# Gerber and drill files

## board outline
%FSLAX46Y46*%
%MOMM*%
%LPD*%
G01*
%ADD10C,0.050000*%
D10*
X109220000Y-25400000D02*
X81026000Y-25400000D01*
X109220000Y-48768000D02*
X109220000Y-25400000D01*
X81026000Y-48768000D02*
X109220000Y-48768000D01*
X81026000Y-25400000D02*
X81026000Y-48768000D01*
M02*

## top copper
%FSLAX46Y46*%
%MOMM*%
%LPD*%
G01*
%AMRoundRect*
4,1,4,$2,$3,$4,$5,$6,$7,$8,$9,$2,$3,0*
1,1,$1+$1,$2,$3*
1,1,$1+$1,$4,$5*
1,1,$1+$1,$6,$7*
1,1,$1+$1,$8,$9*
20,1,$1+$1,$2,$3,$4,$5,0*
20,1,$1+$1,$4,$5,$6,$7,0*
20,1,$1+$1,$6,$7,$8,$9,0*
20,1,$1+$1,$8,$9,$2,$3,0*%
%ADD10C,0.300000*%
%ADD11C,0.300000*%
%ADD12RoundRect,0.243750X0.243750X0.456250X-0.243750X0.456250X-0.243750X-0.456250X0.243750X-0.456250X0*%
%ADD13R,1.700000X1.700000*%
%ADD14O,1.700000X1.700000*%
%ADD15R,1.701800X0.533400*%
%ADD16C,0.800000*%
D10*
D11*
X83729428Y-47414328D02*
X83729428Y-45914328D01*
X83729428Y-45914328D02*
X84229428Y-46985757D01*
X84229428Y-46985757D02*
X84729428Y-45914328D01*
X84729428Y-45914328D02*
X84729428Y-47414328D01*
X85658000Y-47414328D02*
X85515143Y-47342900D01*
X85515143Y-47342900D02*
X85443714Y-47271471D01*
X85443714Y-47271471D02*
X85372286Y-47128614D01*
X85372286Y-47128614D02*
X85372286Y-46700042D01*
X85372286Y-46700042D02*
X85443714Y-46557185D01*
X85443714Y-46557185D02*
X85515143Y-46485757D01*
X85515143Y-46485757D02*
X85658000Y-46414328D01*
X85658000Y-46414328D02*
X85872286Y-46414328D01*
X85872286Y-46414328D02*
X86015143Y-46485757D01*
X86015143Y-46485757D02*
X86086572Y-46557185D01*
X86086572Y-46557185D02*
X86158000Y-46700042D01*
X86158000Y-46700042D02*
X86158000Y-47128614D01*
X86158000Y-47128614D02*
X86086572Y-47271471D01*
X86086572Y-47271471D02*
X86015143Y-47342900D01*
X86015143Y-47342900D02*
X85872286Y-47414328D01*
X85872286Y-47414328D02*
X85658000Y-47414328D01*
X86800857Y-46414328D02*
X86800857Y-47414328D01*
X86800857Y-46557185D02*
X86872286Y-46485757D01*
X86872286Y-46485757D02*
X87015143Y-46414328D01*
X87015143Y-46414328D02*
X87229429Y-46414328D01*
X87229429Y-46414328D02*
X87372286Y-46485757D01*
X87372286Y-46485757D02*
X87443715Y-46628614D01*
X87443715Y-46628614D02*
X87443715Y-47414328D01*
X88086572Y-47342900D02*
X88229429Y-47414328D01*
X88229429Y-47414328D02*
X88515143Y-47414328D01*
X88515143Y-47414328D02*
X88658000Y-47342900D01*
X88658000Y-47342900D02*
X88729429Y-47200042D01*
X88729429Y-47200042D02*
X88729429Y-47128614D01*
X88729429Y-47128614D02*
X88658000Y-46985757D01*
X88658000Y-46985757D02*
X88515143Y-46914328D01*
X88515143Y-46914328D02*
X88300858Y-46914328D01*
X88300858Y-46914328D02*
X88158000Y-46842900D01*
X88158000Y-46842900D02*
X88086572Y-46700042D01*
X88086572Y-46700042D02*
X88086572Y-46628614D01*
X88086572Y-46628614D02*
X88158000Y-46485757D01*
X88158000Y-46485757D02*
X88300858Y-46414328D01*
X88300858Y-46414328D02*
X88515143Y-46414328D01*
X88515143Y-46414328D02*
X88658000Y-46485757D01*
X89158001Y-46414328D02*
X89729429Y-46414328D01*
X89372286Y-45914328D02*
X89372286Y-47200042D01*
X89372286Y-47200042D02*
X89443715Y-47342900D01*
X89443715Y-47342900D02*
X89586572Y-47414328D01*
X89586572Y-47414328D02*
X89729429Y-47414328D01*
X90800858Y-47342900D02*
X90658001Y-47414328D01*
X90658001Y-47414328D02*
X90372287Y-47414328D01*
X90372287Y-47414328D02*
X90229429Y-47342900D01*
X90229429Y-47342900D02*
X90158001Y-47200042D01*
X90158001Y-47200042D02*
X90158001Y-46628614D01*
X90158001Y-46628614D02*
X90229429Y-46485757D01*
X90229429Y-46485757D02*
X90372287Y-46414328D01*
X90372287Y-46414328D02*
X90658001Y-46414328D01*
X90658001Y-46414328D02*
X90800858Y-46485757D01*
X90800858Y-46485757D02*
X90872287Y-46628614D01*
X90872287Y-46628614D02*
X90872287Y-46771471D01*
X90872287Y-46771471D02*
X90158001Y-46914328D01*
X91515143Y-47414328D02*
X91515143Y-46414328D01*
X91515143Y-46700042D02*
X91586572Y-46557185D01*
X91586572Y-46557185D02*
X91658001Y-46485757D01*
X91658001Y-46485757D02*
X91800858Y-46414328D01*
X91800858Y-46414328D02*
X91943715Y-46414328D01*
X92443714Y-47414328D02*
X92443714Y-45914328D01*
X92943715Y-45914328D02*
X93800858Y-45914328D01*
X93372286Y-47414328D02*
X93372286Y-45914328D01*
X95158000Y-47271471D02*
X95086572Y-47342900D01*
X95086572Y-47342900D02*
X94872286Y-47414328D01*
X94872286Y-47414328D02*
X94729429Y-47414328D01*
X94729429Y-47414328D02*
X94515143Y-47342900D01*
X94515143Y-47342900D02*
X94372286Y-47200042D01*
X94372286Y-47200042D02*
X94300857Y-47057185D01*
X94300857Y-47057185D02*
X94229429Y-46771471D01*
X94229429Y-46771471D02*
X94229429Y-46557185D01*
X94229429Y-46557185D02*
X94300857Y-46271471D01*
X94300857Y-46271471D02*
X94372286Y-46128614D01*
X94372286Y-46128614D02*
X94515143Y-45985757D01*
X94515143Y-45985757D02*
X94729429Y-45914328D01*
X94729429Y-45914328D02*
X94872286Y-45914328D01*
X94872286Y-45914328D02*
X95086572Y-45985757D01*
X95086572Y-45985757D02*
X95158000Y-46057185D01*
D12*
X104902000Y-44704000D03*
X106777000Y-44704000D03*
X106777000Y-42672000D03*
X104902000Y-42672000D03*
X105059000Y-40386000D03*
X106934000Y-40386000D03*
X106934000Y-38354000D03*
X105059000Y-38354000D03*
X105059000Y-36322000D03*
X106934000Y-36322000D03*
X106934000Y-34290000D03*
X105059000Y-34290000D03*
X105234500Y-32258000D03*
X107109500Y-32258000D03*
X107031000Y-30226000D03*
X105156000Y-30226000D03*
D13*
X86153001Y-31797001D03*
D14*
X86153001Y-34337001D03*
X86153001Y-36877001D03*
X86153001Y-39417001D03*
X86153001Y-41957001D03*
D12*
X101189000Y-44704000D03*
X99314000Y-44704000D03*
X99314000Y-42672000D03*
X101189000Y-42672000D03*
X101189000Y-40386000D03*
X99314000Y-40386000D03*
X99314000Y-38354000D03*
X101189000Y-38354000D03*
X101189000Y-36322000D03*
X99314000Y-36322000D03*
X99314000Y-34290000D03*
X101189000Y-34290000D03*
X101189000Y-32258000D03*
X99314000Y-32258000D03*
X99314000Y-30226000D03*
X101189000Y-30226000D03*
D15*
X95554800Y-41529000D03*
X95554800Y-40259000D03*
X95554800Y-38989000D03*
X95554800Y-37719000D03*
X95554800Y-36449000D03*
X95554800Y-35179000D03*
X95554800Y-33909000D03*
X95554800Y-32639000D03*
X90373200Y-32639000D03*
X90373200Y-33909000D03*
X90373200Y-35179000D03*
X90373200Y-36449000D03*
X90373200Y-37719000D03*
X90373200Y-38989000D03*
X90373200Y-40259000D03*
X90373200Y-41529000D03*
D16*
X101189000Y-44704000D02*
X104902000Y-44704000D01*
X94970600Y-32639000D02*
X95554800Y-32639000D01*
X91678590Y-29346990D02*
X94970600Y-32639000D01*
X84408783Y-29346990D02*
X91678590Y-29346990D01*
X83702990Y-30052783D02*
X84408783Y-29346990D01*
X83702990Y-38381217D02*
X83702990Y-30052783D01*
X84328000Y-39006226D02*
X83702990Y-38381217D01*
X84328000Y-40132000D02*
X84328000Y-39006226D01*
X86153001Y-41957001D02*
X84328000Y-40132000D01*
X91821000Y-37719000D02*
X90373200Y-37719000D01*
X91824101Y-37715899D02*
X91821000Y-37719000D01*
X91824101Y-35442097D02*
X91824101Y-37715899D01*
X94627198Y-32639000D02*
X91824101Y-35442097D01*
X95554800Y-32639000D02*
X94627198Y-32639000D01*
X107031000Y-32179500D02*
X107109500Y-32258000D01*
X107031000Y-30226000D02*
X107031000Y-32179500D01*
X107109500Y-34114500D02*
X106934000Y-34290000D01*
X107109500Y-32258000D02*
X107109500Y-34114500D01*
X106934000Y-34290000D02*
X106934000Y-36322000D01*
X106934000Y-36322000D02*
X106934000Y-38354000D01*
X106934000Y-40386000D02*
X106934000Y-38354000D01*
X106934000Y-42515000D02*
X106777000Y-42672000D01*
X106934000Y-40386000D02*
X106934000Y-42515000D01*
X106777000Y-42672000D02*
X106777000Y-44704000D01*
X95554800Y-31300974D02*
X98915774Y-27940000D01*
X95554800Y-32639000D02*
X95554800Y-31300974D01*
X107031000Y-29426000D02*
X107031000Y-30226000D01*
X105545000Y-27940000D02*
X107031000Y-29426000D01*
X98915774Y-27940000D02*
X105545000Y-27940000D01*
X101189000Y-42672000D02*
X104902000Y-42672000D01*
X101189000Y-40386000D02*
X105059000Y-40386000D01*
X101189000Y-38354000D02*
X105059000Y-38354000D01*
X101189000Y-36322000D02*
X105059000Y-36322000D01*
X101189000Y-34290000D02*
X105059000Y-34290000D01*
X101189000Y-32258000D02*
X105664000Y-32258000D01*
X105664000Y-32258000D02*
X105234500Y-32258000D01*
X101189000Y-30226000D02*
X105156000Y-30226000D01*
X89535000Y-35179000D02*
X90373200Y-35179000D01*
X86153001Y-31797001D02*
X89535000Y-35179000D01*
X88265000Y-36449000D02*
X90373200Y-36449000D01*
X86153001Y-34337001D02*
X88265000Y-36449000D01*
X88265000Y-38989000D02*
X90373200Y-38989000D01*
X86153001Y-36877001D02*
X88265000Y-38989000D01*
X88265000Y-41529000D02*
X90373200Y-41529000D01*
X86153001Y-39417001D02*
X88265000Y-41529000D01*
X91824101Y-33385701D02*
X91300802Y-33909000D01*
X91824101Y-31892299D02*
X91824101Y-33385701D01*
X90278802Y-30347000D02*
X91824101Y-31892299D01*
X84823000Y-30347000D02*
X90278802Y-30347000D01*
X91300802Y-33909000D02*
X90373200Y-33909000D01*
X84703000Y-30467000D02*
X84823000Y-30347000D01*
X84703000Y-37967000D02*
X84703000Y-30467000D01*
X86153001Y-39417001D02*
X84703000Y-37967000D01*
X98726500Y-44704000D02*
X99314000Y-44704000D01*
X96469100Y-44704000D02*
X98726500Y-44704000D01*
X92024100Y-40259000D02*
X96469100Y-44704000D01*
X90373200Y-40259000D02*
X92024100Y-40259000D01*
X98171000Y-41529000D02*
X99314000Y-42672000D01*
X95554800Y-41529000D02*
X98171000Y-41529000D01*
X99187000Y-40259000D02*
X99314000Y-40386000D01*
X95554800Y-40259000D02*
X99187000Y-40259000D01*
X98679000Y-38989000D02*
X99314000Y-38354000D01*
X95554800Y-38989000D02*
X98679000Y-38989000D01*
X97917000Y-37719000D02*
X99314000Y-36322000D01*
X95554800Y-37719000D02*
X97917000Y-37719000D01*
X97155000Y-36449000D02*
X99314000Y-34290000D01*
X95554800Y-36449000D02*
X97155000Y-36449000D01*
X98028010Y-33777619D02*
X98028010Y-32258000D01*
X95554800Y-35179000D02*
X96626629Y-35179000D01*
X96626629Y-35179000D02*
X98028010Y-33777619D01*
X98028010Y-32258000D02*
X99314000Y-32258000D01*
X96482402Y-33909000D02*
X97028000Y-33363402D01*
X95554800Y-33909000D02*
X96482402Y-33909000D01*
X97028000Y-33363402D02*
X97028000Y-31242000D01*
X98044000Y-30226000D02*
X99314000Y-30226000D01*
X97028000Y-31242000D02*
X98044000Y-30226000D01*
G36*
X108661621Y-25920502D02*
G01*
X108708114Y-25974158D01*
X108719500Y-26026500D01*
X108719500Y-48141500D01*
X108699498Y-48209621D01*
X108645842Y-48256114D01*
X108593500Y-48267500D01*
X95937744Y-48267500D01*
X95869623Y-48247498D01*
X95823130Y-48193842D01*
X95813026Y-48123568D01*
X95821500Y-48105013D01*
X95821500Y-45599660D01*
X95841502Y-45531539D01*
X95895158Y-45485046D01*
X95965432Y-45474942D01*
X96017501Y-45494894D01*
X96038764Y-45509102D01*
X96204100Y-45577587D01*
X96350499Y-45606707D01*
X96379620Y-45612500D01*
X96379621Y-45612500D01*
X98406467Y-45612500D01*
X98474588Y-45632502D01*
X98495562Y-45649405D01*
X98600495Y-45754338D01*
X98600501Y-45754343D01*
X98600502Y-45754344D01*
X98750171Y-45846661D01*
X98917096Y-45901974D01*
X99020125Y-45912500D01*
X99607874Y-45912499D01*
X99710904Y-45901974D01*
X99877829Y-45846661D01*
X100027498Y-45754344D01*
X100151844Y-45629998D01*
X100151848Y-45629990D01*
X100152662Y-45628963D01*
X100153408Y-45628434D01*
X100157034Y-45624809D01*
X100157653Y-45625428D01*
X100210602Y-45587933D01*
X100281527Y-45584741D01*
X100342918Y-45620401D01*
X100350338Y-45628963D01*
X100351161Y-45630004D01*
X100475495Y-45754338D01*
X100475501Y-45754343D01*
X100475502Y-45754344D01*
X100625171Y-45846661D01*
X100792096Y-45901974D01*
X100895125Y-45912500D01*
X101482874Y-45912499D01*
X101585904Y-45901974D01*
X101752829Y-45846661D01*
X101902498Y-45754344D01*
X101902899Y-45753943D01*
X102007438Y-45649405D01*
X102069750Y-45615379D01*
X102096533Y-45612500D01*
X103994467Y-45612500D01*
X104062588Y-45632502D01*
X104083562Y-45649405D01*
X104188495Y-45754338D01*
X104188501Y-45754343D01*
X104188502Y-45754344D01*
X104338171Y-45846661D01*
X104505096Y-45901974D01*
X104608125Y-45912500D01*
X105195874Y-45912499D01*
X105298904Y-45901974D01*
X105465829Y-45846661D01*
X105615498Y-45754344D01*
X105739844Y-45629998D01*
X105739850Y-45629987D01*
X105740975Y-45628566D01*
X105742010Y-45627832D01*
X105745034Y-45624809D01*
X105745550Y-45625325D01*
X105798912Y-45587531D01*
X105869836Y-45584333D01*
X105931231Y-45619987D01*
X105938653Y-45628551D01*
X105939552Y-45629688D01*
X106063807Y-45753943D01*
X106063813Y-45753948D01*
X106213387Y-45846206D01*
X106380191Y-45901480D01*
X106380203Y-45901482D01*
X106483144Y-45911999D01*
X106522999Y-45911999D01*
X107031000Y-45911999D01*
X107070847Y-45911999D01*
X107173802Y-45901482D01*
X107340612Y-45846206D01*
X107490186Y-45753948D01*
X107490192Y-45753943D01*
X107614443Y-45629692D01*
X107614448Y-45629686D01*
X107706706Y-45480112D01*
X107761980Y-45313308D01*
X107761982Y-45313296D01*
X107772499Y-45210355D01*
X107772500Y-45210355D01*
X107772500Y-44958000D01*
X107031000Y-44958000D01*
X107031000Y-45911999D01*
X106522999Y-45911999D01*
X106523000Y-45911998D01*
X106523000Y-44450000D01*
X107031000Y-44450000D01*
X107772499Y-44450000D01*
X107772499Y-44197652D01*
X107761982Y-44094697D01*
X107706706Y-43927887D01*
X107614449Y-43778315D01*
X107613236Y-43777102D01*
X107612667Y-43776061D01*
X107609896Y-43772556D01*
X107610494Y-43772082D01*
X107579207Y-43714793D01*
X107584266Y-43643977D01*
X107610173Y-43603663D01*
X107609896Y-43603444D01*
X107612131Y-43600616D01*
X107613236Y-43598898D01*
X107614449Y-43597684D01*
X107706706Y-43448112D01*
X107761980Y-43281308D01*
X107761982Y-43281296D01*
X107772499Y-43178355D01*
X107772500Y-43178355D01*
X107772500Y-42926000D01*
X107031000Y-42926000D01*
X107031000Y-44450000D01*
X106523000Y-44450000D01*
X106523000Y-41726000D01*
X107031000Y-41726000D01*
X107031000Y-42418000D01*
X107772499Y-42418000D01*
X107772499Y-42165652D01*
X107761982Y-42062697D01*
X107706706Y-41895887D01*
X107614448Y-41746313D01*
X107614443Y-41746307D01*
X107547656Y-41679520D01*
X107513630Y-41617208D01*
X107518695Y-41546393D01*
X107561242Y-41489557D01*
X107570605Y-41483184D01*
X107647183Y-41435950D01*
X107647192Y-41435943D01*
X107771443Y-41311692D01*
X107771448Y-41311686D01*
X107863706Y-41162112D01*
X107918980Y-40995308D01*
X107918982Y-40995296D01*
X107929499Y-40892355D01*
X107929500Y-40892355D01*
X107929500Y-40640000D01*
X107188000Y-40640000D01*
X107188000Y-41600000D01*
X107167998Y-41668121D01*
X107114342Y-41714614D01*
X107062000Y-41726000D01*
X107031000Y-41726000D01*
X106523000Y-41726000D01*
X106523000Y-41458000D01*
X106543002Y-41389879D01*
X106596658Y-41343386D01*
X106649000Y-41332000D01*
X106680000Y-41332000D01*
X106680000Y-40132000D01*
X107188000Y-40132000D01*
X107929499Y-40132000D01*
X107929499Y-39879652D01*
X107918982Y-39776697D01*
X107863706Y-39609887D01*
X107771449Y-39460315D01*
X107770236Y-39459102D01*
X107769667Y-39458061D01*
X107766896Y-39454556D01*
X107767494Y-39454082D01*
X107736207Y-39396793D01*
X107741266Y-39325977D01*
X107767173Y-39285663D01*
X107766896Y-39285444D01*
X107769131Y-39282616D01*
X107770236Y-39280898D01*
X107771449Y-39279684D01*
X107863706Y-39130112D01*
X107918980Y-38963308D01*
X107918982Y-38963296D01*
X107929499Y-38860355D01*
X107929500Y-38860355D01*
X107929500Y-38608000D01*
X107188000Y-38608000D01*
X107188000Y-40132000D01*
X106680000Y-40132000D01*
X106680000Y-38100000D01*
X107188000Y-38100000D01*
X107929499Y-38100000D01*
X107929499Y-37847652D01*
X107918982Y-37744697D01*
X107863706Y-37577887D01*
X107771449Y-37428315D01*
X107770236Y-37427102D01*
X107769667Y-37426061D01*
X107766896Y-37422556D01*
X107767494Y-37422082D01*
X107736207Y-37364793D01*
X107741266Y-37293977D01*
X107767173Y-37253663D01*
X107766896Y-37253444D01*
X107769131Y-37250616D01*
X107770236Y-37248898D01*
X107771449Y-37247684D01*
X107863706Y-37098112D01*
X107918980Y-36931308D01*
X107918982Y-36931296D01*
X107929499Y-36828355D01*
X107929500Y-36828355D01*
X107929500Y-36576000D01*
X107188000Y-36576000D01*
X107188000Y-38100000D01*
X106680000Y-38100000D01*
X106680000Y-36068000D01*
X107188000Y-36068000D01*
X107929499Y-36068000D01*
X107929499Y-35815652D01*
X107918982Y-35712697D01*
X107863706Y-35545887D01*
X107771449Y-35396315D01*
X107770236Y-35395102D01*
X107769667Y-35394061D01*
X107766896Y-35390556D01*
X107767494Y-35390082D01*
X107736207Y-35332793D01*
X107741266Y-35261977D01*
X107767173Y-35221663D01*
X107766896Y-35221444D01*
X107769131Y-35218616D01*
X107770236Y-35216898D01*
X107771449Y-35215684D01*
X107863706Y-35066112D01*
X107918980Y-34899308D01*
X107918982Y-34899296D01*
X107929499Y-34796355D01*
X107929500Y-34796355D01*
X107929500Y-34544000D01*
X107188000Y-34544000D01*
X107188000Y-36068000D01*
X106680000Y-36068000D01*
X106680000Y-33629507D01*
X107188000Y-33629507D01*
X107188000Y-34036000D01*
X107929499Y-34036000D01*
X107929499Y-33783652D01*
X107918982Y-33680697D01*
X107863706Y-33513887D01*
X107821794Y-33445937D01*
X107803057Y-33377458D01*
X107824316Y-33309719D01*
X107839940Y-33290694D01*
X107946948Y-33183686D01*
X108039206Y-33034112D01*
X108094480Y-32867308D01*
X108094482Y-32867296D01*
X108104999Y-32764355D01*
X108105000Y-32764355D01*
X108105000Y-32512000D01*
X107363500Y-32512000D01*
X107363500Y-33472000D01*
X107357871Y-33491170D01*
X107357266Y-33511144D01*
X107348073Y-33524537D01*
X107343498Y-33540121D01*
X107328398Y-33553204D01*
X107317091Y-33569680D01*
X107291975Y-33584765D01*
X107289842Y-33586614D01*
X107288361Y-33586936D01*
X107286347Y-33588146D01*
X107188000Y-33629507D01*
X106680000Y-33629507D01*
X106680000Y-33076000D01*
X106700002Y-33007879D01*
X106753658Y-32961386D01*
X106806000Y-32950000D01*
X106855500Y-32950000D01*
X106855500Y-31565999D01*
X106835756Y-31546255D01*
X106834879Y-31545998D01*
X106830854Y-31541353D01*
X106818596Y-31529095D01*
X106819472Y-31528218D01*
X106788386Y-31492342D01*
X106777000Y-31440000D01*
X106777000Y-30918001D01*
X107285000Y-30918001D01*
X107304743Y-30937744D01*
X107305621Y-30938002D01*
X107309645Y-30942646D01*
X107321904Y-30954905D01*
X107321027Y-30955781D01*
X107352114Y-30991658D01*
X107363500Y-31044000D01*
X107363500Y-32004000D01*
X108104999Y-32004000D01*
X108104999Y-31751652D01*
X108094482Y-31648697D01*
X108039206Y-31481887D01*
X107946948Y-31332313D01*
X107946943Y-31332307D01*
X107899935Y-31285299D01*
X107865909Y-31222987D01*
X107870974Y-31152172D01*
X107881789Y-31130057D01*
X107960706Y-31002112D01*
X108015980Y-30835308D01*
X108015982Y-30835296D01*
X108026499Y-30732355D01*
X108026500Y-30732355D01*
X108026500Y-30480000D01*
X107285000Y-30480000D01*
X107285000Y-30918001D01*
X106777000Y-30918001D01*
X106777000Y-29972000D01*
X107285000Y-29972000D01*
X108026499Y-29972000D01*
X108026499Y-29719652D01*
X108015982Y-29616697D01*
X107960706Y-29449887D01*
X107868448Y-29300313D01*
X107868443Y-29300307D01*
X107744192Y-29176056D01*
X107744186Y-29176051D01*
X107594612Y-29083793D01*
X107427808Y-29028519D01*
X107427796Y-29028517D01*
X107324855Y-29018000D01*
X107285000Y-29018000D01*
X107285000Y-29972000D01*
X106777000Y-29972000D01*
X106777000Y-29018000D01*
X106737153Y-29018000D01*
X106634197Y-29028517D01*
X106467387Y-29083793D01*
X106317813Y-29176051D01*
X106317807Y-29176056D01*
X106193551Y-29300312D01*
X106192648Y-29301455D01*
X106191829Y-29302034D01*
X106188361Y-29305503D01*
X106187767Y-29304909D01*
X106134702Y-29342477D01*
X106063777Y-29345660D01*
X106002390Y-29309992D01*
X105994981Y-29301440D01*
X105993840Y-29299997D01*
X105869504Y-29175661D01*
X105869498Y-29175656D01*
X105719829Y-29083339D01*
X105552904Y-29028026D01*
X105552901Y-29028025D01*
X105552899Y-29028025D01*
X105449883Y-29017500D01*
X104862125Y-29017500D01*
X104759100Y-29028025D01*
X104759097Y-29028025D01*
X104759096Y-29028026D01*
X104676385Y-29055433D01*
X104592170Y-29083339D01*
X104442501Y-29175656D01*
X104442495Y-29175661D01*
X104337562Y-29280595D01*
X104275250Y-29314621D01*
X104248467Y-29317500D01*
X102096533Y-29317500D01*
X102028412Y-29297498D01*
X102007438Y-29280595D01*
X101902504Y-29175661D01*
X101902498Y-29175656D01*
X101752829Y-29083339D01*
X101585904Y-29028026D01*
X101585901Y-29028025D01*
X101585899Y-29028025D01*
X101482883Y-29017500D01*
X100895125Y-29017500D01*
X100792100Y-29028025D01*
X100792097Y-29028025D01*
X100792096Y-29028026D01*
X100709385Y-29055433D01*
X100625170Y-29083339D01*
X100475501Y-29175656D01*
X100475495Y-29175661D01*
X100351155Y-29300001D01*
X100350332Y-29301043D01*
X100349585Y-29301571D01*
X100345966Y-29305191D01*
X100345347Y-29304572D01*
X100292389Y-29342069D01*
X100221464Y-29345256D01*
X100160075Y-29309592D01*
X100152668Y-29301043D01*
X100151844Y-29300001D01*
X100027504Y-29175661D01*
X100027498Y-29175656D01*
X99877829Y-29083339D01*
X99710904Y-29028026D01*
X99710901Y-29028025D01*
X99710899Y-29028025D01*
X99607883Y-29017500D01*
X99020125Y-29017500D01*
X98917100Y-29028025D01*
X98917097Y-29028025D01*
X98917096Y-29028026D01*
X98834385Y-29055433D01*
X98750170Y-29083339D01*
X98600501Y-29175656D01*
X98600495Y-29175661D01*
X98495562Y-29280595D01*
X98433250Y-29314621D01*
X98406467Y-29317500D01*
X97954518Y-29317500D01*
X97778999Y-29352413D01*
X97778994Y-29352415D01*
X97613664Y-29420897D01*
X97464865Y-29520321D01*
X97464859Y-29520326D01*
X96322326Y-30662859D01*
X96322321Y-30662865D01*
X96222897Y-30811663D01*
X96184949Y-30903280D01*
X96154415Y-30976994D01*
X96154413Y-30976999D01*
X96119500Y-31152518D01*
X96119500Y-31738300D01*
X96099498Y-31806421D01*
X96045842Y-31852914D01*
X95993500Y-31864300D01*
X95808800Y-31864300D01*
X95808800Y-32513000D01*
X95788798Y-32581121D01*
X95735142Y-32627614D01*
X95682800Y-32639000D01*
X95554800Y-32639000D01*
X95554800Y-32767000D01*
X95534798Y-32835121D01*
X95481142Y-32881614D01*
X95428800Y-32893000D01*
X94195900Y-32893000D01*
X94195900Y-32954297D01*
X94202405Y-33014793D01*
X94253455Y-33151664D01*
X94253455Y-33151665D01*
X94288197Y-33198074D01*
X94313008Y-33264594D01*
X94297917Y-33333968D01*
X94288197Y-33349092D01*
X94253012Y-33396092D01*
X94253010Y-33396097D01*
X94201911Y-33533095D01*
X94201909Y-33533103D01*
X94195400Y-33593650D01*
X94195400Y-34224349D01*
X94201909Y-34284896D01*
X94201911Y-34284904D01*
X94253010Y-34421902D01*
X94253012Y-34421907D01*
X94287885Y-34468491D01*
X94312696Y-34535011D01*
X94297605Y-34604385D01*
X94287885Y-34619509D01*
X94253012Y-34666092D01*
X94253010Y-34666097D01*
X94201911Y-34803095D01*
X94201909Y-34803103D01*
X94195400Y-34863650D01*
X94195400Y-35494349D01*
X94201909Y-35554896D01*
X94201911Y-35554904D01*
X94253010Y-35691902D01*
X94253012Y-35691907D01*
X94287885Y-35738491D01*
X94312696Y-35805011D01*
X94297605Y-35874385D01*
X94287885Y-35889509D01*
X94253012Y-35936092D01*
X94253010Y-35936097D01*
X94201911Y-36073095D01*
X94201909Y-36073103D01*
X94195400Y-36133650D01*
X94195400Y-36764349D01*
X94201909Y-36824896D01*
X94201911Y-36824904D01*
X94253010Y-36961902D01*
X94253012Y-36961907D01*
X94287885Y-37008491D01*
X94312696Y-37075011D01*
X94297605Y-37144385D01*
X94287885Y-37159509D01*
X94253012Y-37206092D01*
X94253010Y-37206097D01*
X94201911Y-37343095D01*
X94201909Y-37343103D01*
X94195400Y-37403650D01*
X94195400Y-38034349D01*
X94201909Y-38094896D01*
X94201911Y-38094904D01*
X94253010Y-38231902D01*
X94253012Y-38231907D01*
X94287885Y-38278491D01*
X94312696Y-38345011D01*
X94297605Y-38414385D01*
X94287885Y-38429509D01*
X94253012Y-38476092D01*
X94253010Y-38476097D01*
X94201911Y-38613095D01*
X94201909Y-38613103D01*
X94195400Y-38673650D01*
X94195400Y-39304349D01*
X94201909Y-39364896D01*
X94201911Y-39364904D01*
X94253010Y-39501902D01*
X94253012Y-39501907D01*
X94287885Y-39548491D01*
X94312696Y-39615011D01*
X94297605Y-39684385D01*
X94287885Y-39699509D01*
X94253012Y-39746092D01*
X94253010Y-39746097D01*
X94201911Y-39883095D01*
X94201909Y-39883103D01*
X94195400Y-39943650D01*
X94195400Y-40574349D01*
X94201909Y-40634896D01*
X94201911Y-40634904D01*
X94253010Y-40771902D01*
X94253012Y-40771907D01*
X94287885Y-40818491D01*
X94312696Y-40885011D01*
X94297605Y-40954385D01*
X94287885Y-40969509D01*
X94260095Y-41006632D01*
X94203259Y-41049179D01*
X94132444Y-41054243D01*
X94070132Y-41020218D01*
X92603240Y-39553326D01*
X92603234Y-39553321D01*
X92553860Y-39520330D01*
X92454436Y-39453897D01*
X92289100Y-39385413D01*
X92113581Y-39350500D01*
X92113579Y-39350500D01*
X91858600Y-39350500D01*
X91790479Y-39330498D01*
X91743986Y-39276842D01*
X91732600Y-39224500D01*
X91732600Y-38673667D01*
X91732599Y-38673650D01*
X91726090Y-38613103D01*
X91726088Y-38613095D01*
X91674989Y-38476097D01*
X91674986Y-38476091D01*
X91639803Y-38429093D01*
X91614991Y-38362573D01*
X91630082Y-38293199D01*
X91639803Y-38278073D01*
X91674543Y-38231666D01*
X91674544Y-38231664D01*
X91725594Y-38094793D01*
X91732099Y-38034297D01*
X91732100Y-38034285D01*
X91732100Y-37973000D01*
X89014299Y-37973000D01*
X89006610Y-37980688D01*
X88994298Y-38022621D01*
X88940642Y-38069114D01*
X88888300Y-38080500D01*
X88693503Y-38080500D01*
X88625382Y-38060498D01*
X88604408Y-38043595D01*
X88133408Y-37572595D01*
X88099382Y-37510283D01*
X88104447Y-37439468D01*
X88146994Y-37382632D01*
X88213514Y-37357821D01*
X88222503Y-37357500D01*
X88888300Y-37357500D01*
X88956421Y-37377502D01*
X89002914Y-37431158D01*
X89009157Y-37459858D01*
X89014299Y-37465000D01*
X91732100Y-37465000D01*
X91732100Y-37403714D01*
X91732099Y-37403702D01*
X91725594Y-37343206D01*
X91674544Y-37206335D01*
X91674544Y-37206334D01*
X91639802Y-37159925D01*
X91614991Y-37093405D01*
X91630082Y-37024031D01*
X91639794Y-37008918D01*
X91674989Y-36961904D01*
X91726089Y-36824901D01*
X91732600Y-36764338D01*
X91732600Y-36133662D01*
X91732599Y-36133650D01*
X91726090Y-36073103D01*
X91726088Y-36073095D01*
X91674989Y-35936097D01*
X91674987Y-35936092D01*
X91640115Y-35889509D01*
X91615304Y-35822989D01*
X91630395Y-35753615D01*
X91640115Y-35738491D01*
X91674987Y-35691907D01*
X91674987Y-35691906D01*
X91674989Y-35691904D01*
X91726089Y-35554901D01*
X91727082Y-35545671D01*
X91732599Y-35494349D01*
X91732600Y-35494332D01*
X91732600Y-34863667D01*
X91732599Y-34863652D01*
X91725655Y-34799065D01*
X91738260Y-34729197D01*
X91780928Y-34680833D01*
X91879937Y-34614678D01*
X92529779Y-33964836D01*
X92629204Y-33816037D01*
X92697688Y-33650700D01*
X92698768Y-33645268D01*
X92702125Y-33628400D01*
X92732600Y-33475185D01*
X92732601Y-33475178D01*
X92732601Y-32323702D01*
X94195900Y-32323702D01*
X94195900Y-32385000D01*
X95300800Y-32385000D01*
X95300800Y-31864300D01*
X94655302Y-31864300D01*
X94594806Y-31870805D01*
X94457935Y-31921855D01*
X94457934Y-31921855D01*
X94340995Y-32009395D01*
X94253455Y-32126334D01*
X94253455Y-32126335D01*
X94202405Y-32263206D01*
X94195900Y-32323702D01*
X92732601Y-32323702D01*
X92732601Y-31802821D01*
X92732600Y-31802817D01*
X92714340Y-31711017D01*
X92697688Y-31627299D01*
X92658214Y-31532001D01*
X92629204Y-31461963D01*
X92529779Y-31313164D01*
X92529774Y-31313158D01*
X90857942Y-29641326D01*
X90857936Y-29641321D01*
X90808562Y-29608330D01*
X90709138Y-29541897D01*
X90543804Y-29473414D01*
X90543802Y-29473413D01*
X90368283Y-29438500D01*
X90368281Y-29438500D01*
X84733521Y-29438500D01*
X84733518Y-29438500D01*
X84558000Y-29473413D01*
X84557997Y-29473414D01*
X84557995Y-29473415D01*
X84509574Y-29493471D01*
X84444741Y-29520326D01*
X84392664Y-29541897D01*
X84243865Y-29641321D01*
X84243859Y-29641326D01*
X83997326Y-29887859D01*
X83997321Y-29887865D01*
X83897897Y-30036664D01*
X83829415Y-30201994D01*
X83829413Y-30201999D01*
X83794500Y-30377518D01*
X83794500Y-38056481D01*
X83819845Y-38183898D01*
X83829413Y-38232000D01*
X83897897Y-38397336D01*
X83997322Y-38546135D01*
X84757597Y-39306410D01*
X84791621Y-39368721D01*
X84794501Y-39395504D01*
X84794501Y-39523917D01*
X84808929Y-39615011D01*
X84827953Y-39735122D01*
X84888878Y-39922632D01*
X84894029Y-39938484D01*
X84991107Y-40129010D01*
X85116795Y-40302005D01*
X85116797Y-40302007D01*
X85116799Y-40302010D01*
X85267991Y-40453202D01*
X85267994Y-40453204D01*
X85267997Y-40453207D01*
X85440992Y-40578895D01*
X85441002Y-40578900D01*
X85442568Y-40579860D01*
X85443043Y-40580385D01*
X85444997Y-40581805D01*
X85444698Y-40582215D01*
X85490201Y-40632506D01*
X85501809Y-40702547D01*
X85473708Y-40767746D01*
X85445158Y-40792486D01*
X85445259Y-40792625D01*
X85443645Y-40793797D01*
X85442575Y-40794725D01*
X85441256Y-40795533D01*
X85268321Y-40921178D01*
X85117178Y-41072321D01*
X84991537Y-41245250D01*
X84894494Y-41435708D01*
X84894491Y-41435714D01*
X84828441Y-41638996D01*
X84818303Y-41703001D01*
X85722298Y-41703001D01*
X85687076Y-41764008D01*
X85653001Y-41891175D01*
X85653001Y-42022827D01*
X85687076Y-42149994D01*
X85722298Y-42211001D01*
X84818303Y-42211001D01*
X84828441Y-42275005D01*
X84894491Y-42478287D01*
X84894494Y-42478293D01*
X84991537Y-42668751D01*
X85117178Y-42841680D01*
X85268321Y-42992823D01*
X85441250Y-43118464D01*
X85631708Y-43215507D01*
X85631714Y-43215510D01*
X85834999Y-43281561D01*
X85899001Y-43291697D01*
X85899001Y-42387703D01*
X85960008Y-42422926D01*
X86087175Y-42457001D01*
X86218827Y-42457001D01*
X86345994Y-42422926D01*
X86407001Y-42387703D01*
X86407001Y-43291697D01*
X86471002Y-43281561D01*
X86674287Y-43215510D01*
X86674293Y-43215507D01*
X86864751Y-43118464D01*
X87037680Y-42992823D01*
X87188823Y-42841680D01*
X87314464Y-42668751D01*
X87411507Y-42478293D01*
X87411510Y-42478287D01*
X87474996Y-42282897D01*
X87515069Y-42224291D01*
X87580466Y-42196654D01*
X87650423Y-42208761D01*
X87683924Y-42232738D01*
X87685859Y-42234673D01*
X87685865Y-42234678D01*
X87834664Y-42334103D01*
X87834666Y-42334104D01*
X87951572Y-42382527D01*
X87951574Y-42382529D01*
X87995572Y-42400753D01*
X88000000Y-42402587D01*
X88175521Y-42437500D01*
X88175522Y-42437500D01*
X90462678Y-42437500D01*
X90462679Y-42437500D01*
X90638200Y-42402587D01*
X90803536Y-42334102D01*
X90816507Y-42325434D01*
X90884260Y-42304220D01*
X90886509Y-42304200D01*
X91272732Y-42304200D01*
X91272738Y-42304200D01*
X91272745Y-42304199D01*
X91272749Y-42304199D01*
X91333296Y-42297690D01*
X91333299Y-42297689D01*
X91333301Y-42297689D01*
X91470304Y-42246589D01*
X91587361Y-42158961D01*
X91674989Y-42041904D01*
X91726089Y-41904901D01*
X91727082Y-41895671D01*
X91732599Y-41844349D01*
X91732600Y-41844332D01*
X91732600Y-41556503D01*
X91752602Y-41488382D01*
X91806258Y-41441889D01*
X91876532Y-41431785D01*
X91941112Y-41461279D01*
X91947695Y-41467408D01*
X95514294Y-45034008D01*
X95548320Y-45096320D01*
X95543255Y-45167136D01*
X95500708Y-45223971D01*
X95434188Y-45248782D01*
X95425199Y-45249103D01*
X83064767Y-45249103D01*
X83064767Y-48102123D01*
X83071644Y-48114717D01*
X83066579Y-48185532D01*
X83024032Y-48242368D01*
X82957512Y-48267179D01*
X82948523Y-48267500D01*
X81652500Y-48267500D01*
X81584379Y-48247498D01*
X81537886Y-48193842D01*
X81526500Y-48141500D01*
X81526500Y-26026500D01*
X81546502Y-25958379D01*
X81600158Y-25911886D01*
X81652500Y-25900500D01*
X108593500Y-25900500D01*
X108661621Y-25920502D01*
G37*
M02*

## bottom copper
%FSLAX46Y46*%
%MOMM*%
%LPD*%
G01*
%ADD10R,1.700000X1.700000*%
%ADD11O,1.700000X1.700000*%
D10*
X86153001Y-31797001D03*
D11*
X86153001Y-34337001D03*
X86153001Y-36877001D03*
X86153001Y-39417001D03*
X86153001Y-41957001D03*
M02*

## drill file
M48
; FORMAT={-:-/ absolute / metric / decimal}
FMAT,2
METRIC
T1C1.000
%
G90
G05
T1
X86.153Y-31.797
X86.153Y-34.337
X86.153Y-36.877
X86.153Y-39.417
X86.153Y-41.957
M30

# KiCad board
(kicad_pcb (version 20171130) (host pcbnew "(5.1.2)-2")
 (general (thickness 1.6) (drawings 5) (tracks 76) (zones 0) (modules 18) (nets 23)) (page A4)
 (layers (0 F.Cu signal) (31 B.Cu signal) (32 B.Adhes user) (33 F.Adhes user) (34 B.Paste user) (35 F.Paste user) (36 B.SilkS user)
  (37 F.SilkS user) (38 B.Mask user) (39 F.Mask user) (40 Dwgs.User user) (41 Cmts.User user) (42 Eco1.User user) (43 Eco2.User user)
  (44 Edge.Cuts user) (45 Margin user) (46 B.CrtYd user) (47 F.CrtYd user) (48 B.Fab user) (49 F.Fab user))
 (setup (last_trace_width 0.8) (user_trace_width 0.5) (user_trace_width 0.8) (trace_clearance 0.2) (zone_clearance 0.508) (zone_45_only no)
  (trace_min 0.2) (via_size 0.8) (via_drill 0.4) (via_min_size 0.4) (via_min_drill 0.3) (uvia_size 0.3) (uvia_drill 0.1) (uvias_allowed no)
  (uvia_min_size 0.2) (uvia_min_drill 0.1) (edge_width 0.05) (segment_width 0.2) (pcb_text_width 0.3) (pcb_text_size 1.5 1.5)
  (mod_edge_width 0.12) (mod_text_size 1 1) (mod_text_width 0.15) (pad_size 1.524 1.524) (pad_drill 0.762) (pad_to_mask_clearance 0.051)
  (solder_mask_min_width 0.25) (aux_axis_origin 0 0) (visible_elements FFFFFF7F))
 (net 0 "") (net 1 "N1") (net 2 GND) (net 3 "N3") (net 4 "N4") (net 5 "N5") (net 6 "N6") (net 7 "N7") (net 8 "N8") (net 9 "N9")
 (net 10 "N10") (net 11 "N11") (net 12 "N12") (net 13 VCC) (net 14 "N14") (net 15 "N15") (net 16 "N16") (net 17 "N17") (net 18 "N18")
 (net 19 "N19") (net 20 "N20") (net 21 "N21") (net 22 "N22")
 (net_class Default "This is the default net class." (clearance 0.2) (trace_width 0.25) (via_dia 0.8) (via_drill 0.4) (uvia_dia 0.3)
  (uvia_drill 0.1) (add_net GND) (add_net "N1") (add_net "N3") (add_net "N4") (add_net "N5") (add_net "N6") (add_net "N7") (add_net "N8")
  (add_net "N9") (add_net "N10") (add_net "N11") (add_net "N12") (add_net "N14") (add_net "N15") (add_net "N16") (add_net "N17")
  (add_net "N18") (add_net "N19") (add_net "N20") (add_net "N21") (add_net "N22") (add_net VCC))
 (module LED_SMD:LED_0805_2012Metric (layer F.Cu) (at 105.8395 44.704 180)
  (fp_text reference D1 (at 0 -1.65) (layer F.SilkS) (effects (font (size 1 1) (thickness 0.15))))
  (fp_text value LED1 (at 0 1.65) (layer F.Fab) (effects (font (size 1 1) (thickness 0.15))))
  (pad 2 smd roundrect (at 0.9375 0 180) (size 0.975 1.4) (layers F.Cu F.Paste F.Mask) (roundrect_rratio 0.25) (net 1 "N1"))
  (pad 1 smd roundrect (at -0.9375 0 180) (size 0.975 1.4) (layers F.Cu F.Paste F.Mask) (roundrect_rratio 0.25) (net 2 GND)))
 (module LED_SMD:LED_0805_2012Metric (layer F.Cu) (at 105.8395 42.672 180)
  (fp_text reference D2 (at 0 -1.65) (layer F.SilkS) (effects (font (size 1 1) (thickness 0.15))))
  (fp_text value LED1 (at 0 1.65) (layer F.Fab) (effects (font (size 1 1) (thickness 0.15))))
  (pad 1 smd roundrect (at -0.9375 0 180) (size 0.975 1.4) (layers F.Cu F.Paste F.Mask) (roundrect_rratio 0.25) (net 2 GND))
  (pad 2 smd roundrect (at 0.9375 0 180) (size 0.975 1.4) (layers F.Cu F.Paste F.Mask) (roundrect_rratio 0.25) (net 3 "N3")))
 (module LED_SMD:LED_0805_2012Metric (layer F.Cu) (at 105.9965 40.386 180)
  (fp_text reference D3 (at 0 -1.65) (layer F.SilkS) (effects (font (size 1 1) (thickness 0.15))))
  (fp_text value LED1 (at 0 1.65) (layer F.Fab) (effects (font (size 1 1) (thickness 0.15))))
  (pad 2 smd roundrect (at 0.9375 0 180) (size 0.975 1.4) (layers F.Cu F.Paste F.Mask) (roundrect_rratio 0.25) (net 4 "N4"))
  (pad 1 smd roundrect (at -0.9375 0 180) (size 0.975 1.4) (layers F.Cu F.Paste F.Mask) (roundrect_rratio 0.25) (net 2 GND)))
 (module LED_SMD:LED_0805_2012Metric (layer F.Cu) (at 105.9965 38.354 180)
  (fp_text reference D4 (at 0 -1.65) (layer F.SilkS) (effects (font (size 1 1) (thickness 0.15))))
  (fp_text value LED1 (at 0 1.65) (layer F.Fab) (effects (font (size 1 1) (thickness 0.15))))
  (pad 1 smd roundrect (at -0.9375 0 180) (size 0.975 1.4) (layers F.Cu F.Paste F.Mask) (roundrect_rratio 0.25) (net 2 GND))
  (pad 2 smd roundrect (at 0.9375 0 180) (size 0.975 1.4) (layers F.Cu F.Paste F.Mask) (roundrect_rratio 0.25) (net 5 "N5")))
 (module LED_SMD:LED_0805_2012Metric (layer F.Cu) (at 105.9965 36.322 180)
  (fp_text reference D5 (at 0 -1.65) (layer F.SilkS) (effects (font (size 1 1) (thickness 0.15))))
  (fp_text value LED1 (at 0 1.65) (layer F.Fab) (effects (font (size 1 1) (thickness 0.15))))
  (pad 2 smd roundrect (at 0.9375 0 180) (size 0.975 1.4) (layers F.Cu F.Paste F.Mask) (roundrect_rratio 0.25) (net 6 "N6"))
  (pad 1 smd roundrect (at -0.9375 0 180) (size 0.975 1.4) (layers F.Cu F.Paste F.Mask) (roundrect_rratio 0.25) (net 2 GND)))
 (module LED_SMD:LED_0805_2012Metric (layer F.Cu) (at 105.9965 34.29 180)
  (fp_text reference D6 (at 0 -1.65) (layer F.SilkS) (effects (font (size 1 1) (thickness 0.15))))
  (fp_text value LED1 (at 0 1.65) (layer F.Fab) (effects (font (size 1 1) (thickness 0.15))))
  (pad 1 smd roundrect (at -0.9375 0 180) (size 0.975 1.4) (layers F.Cu F.Paste F.Mask) (roundrect_rratio 0.25) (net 2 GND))
  (pad 2 smd roundrect (at 0.9375 0 180) (size 0.975 1.4) (layers F.Cu F.Paste F.Mask) (roundrect_rratio 0.25) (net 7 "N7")))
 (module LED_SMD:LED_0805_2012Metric (layer F.Cu) (at 106.172 32.258 180)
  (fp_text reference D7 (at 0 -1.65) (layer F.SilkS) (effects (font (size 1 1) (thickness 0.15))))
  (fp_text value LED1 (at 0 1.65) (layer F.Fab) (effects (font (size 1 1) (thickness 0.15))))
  (pad 2 smd roundrect (at 0.9375 0 180) (size 0.975 1.4) (layers F.Cu F.Paste F.Mask) (roundrect_rratio 0.25) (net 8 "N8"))
  (pad 1 smd roundrect (at -0.9375 0 180) (size 0.975 1.4) (layers F.Cu F.Paste F.Mask) (roundrect_rratio 0.25) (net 2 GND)))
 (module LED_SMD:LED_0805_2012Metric (layer F.Cu) (at 106.0935 30.226 180)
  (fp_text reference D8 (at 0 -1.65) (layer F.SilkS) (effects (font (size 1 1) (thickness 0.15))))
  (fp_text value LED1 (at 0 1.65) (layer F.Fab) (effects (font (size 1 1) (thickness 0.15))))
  (pad 1 smd roundrect (at -0.9375 0 180) (size 0.975 1.4) (layers F.Cu F.Paste F.Mask) (roundrect_rratio 0.25) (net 2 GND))
  (pad 2 smd roundrect (at 0.9375 0 180) (size 0.975 1.4) (layers F.Cu F.Paste F.Mask) (roundrect_rratio 0.25) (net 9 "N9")))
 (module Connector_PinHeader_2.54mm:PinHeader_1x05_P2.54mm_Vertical (layer F.Cu) (at 86.153001 31.797001)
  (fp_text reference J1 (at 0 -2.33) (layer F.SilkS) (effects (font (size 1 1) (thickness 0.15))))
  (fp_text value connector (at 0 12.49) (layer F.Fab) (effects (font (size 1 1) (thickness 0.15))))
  (pad 1 thru_hole rect (at 0 0) (size 1.7 1.7) (drill 1) (layers *.Cu *.Mask) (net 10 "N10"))
  (pad 2 thru_hole oval (at 0 2.54) (size 1.7 1.7) (drill 1) (layers *.Cu *.Mask) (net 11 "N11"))
  (pad 3 thru_hole oval (at 0 5.08) (size 1.7 1.7) (drill 1) (layers *.Cu *.Mask) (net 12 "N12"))
  (pad 4 thru_hole oval (at 0 7.62) (size 1.7 1.7) (drill 1) (layers *.Cu *.Mask) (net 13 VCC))
  (pad 5 thru_hole oval (at 0 10.16) (size 1.7 1.7) (drill 1) (layers *.Cu *.Mask) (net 2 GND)))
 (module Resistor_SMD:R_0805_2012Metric (layer F.Cu) (at 100.2515 44.704 180)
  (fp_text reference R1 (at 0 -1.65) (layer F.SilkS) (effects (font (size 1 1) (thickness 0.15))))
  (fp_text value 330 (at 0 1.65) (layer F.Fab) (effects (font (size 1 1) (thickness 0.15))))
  (pad 1 smd roundrect (at -0.9375 0 180) (size 0.975 1.4) (layers F.Cu F.Paste F.Mask) (roundrect_rratio 0.25) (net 1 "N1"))
  (pad 2 smd roundrect (at 0.9375 0 180) (size 0.975 1.4) (layers F.Cu F.Paste F.Mask) (roundrect_rratio 0.25) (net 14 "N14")))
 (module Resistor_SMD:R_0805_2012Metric (layer F.Cu) (at 100.2515 42.672 180)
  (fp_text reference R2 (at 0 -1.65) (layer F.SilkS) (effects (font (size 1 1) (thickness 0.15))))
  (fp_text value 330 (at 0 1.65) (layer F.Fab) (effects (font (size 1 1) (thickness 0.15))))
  (pad 2 smd roundrect (at 0.9375 0 180) (size 0.975 1.4) (layers F.Cu F.Paste F.Mask) (roundrect_rratio 0.25) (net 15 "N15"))
  (pad 1 smd roundrect (at -0.9375 0 180) (size 0.975 1.4) (layers F.Cu F.Paste F.Mask) (roundrect_rratio 0.25) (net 3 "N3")))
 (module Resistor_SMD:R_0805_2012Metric (layer F.Cu) (at 100.2515 40.386 180)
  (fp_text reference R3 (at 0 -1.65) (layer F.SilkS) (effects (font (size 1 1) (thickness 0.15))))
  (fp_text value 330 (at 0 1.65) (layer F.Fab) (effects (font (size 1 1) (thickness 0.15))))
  (pad 1 smd roundrect (at -0.9375 0 180) (size 0.975 1.4) (layers F.Cu F.Paste F.Mask) (roundrect_rratio 0.25) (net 4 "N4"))
  (pad 2 smd roundrect (at 0.9375 0 180) (size 0.975 1.4) (layers F.Cu F.Paste F.Mask) (roundrect_rratio 0.25) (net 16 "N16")))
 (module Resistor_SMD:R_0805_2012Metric (layer F.Cu) (at 100.2515 38.354 180)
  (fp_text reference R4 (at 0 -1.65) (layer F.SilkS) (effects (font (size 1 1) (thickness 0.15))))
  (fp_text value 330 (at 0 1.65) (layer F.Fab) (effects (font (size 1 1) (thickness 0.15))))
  (pad 2 smd roundrect (at 0.9375 0 180) (size 0.975 1.4) (layers F.Cu F.Paste F.Mask) (roundrect_rratio 0.25) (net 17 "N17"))
  (pad 1 smd roundrect (at -0.9375 0 180) (size 0.975 1.4) (layers F.Cu F.Paste F.Mask) (roundrect_rratio 0.25) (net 5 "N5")))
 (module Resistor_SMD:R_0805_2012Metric (layer F.Cu) (at 100.2515 36.322 180)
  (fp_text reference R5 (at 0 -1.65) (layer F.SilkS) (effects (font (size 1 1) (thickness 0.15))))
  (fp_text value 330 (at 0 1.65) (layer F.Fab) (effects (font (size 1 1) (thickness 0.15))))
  (pad 1 smd roundrect (at -0.9375 0 180) (size 0.975 1.4) (layers F.Cu F.Paste F.Mask) (roundrect_rratio 0.25) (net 6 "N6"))
  (pad 2 smd roundrect (at 0.9375 0 180) (size 0.975 1.4) (layers F.Cu F.Paste F.Mask) (roundrect_rratio 0.25) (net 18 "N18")))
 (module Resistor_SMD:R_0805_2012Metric (layer F.Cu) (at 100.2515 34.29 180)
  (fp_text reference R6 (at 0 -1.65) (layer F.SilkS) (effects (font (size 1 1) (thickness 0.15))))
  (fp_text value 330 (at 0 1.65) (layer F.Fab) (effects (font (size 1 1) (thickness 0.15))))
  (pad 2 smd roundrect (at 0.9375 0 180) (size 0.975 1.4) (layers F.Cu F.Paste F.Mask) (roundrect_rratio 0.25) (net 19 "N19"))
  (pad 1 smd roundrect (at -0.9375 0 180) (size 0.975 1.4) (layers F.Cu F.Paste F.Mask) (roundrect_rratio 0.25) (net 7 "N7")))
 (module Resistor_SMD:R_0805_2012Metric (layer F.Cu) (at 100.2515 32.258 180)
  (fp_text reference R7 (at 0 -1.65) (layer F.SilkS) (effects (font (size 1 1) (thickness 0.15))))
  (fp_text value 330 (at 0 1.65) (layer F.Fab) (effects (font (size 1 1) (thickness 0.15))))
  (pad 1 smd roundrect (at -0.9375 0 180) (size 0.975 1.4) (layers F.Cu F.Paste F.Mask) (roundrect_rratio 0.25) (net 8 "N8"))
  (pad 2 smd roundrect (at 0.9375 0 180) (size 0.975 1.4) (layers F.Cu F.Paste F.Mask) (roundrect_rratio 0.25) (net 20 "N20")))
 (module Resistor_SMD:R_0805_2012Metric (layer F.Cu) (at 100.2515 30.226 180)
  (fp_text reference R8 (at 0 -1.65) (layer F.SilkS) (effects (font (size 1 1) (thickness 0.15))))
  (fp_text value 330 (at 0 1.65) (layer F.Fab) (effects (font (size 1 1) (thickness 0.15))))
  (pad 2 smd roundrect (at 0.9375 0 180) (size 0.975 1.4) (layers F.Cu F.Paste F.Mask) (roundrect_rratio 0.25) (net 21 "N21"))
  (pad 1 smd roundrect (at -0.9375 0 180) (size 0.975 1.4) (layers F.Cu F.Paste F.Mask) (roundrect_rratio 0.25) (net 9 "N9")))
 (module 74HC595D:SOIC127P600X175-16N (layer F.Cu) (at 92.964 37.084 180)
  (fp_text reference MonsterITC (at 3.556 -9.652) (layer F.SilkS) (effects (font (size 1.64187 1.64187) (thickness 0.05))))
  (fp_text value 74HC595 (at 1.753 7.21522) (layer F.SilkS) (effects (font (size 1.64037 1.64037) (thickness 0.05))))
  (pad 1 smd rect (at -2.5908 -4.445 180) (size 1.7018 0.5334) (layers F.Cu F.Paste F.Mask) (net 15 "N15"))
  (pad 2 smd rect (at -2.5908 -3.175 180) (size 1.7018 0.5334) (layers F.Cu F.Paste F.Mask) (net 16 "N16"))
  (pad 3 smd rect (at -2.5908 -1.905 180) (size 1.7018 0.5334) (layers F.Cu F.Paste F.Mask) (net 17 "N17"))
  (pad 4 smd rect (at -2.5908 -0.635 180) (size 1.7018 0.5334) (layers F.Cu F.Paste F.Mask) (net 18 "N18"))
  (pad 5 smd rect (at -2.5908 0.635 180) (size 1.7018 0.5334) (layers F.Cu F.Paste F.Mask) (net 19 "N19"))
  (pad 6 smd rect (at -2.5908 1.905 180) (size 1.7018 0.5334) (layers F.Cu F.Paste F.Mask) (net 20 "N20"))
  (pad 7 smd rect (at -2.5908 3.175 180) (size 1.7018 0.5334) (layers F.Cu F.Paste F.Mask) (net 21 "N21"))
  (pad 8 smd rect (at -2.5908 4.445 180) (size 1.7018 0.5334) (layers F.Cu F.Paste F.Mask) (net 2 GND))
  (pad 9 smd rect (at 2.5908 4.445 180) (size 1.7018 0.5334) (layers F.Cu F.Paste F.Mask) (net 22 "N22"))
  (pad 10 smd rect (at 2.5908 3.175 180) (size 1.7018 0.5334) (layers F.Cu F.Paste F.Mask) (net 13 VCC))
  (pad 11 smd rect (at 2.5908 1.905 180) (size 1.7018 0.5334) (layers F.Cu F.Paste F.Mask) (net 10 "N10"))
  (pad 12 smd rect (at 2.5908 0.635 180) (size 1.7018 0.5334) (layers F.Cu F.Paste F.Mask) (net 11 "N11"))
  (pad 13 smd rect (at 2.5908 -0.635 180) (size 1.7018 0.5334) (layers F.Cu F.Paste F.Mask) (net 2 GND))
  (pad 14 smd rect (at 2.5908 -1.905 180) (size 1.7018 0.5334) (layers F.Cu F.Paste F.Mask) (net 12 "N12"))
  (pad 15 smd rect (at 2.5908 -3.175 180) (size 1.7018 0.5334) (layers F.Cu F.Paste F.Mask) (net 14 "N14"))
  (pad 16 smd rect (at 2.5908 -4.445 180) (size 1.7018 0.5334) (layers F.Cu F.Paste F.Mask) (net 13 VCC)))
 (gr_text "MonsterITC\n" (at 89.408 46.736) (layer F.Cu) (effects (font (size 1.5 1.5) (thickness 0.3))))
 (gr_line (start 109.22 25.4) (end 81.026 25.4) (layer Edge.Cuts) (width 0.05))
 (gr_line (start 109.22 48.768) (end 109.22 25.4) (layer Edge.Cuts) (width 0.05))
 (gr_line (start 81.026 48.768) (end 109.22 48.768) (layer Edge.Cuts) (width 0.05))
 (gr_line (start 81.026 25.4) (end 81.026 48.768) (layer Edge.Cuts) (width 0.05))
 (segment (start 101.189 44.704) (end 104.902 44.704) (width 0.8) (layer F.Cu) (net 1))
 (segment (start 94.9706 32.639) (end 95.5548 32.639) (width 0.8) (layer F.Cu) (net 2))
 (segment (start 91.67859 29.34699) (end 94.9706 32.639) (width 0.8) (layer F.Cu) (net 2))
 (segment (start 84.408783 29.34699) (end 91.67859 29.34699) (width 0.8) (layer F.Cu) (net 2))
 (segment (start 83.70299 30.052783) (end 84.408783 29.34699) (width 0.8) (layer F.Cu) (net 2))
 (segment (start 83.70299 38.381217) (end 83.70299 30.052783) (width 0.8) (layer F.Cu) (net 2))
 (segment (start 84.328 39.006226) (end 83.70299 38.381217) (width 0.8) (layer F.Cu) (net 2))
 (segment (start 84.328 40.132) (end 84.328 39.006226) (width 0.8) (layer F.Cu) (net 2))
 (segment (start 86.153001 41.957001) (end 84.328 40.132) (width 0.8) (layer F.Cu) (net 2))
 (segment (start 91.821 37.719) (end 90.3732 37.719) (width 0.8) (layer F.Cu) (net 2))
 (segment (start 91.824101 37.715899) (end 91.821 37.719) (width 0.8) (layer F.Cu) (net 2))
 (segment (start 91.824101 35.442097) (end 91.824101 37.715899) (width 0.8) (layer F.Cu) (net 2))
 (segment (start 94.627198 32.639) (end 91.824101 35.442097) (width 0.8) (layer F.Cu) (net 2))
 (segment (start 95.5548 32.639) (end 94.627198 32.639) (width 0.8) (layer F.Cu) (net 2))
 (segment (start 107.031 32.1795) (end 107.1095 32.258) (width 0.8) (layer F.Cu) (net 2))
 (segment (start 107.031 30.226) (end 107.031 32.1795) (width 0.8) (layer F.Cu) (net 2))
 (segment (start 107.1095 34.1145) (end 106.934 34.29) (width 0.8) (layer F.Cu) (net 2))
 (segment (start 107.1095 32.258) (end 107.1095 34.1145) (width 0.8) (layer F.Cu) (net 2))
 (segment (start 106.934 34.29) (end 106.934 36.322) (width 0.8) (layer F.Cu) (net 2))
 (segment (start 106.934 36.322) (end 106.934 38.354) (width 0.8) (layer F.Cu) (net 2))
 (segment (start 106.934 40.386) (end 106.934 38.354) (width 0.8) (layer F.Cu) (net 2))
 (segment (start 106.934 42.515) (end 106.777 42.672) (width 0.8) (layer F.Cu) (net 2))
 (segment (start 106.934 40.386) (end 106.934 42.515) (width 0.8) (layer F.Cu) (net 2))
 (segment (start 106.777 42.672) (end 106.777 44.704) (width 0.8) (layer F.Cu) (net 2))
 (segment (start 95.5548 31.300974) (end 98.915774 27.94) (width 0.8) (layer F.Cu) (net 2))
 (segment (start 95.5548 32.639) (end 95.5548 31.300974) (width 0.8) (layer F.Cu) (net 2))
 (segment (start 107.031 29.426) (end 107.031 30.226) (width 0.8) (layer F.Cu) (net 2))
 (segment (start 105.545 27.94) (end 107.031 29.426) (width 0.8) (layer F.Cu) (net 2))
 (segment (start 98.915774 27.94) (end 105.545 27.94) (width 0.8) (layer F.Cu) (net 2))
 (segment (start 101.189 42.672) (end 104.902 42.672) (width 0.8) (layer F.Cu) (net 3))
 (segment (start 101.189 40.386) (end 105.059 40.386) (width 0.8) (layer F.Cu) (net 4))
 (segment (start 101.189 38.354) (end 105.059 38.354) (width 0.8) (layer F.Cu) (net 5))
 (segment (start 101.189 36.322) (end 105.059 36.322) (width 0.8) (layer F.Cu) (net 6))
 (segment (start 101.189 34.29) (end 105.059 34.29) (width 0.8) (layer F.Cu) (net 7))
 (segment (start 101.189 32.258) (end 105.664 32.258) (width 0.8) (layer F.Cu) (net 8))
 (segment (start 105.664 32.258) (end 105.2345 32.258) (width 0.8) (layer F.Cu) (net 8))
 (segment (start 101.189 30.226) (end 105.156 30.226) (width 0.8) (layer F.Cu) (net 9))
 (segment (start 89.535 35.179) (end 90.3732 35.179) (width 0.8) (layer F.Cu) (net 10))
 (segment (start 86.153001 31.797001) (end 89.535 35.179) (width 0.8) (layer F.Cu) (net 10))
 (segment (start 88.265 36.449) (end 90.3732 36.449) (width 0.8) (layer F.Cu) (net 11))
 (segment (start 86.153001 34.337001) (end 88.265 36.449) (width 0.8) (layer F.Cu) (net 11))
 (segment (start 88.265 38.989) (end 90.3732 38.989) (width 0.8) (layer F.Cu) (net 12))
 (segment (start 86.153001 36.877001) (end 88.265 38.989) (width 0.8) (layer F.Cu) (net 12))
 (segment (start 88.265 41.529) (end 90.3732 41.529) (width 0.8) (layer F.Cu) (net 13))
 (segment (start 86.153001 39.417001) (end 88.265 41.529) (width 0.8) (layer F.Cu) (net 13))
 (segment (start 91.824101 33.385701) (end 91.300802 33.909) (width 0.8) (layer F.Cu) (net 13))
 (segment (start 91.824101 31.892299) (end 91.824101 33.385701) (width 0.8) (layer F.Cu) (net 13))
 (segment (start 90.278802 30.347) (end 91.824101 31.892299) (width 0.8) (layer F.Cu) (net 13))
 (segment (start 84.823 30.347) (end 90.278802 30.347) (width 0.8) (layer F.Cu) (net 13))
 (segment (start 91.300802 33.909) (end 90.3732 33.909) (width 0.8) (layer F.Cu) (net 13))
 (segment (start 84.703 30.467) (end 84.823 30.347) (width 0.8) (layer F.Cu) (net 13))
 (segment (start 84.703 37.967) (end 84.703 30.467) (width 0.8) (layer F.Cu) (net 13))
 (segment (start 86.153001 39.417001) (end 84.703 37.967) (width 0.8) (layer F.Cu) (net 13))
 (segment (start 98.7265 44.704) (end 99.314 44.704) (width 0.8) (layer F.Cu) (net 14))
 (segment (start 96.4691 44.704) (end 98.7265 44.704) (width 0.8) (layer F.Cu) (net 14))
 (segment (start 92.0241 40.259) (end 96.4691 44.704) (width 0.8) (layer F.Cu) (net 14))
 (segment (start 90.3732 40.259) (end 92.0241 40.259) (width 0.8) (layer F.Cu) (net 14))
 (segment (start 98.171 41.529) (end 99.314 42.672) (width 0.8) (layer F.Cu) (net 15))
 (segment (start 95.5548 41.529) (end 98.171 41.529) (width 0.8) (layer F.Cu) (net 15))
 (segment (start 99.187 40.259) (end 99.314 40.386) (width 0.8) (layer F.Cu) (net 16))
 (segment (start 95.5548 40.259) (end 99.187 40.259) (width 0.8) (layer F.Cu) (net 16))
 (segment (start 98.679 38.989) (end 99.314 38.354) (width 0.8) (layer F.Cu) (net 17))
 (segment (start 95.5548 38.989) (end 98.679 38.989) (width 0.8) (layer F.Cu) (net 17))
 (segment (start 97.917 37.719) (end 99.314 36.322) (width 0.8) (layer F.Cu) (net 18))
 (segment (start 95.5548 37.719) (end 97.917 37.719) (width 0.8) (layer F.Cu) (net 18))
 (segment (start 97.155 36.449) (end 99.314 34.29) (width 0.8) (layer F.Cu) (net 19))
 (segment (start 95.5548 36.449) (end 97.155 36.449) (width 0.8) (layer F.Cu) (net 19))
 (segment (start 98.02801 33.777619) (end 98.02801 32.258) (width 0.8) (layer F.Cu) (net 20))
 (segment (start 95.5548 35.179) (end 96.626629 35.179) (width 0.8) (layer F.Cu) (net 20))
 (segment (start 96.626629 35.179) (end 98.02801 33.777619) (width 0.8) (layer F.Cu) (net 20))
 (segment (start 98.02801 32.258) (end 99.314 32.258) (width 0.8) (layer F.Cu) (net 20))
 (segment (start 96.482402 33.909) (end 97.028 33.363402) (width 0.8) (layer F.Cu) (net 21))
 (segment (start 95.5548 33.909) (end 96.482402 33.909) (width 0.8) (layer F.Cu) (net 21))
 (segment (start 97.028 33.363402) (end 97.028 31.242) (width 0.8) (layer F.Cu) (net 21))
 (segment (start 98.044 30.226) (end 99.314 30.226) (width 0.8) (layer F.Cu) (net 21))
 (segment (start 97.028 31.242) (end 98.044 30.226) (width 0.8) (layer F.Cu) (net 21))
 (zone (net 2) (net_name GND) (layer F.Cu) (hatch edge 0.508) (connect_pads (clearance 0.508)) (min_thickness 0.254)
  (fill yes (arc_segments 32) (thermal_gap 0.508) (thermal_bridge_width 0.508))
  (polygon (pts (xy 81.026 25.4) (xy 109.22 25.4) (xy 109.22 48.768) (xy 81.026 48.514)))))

